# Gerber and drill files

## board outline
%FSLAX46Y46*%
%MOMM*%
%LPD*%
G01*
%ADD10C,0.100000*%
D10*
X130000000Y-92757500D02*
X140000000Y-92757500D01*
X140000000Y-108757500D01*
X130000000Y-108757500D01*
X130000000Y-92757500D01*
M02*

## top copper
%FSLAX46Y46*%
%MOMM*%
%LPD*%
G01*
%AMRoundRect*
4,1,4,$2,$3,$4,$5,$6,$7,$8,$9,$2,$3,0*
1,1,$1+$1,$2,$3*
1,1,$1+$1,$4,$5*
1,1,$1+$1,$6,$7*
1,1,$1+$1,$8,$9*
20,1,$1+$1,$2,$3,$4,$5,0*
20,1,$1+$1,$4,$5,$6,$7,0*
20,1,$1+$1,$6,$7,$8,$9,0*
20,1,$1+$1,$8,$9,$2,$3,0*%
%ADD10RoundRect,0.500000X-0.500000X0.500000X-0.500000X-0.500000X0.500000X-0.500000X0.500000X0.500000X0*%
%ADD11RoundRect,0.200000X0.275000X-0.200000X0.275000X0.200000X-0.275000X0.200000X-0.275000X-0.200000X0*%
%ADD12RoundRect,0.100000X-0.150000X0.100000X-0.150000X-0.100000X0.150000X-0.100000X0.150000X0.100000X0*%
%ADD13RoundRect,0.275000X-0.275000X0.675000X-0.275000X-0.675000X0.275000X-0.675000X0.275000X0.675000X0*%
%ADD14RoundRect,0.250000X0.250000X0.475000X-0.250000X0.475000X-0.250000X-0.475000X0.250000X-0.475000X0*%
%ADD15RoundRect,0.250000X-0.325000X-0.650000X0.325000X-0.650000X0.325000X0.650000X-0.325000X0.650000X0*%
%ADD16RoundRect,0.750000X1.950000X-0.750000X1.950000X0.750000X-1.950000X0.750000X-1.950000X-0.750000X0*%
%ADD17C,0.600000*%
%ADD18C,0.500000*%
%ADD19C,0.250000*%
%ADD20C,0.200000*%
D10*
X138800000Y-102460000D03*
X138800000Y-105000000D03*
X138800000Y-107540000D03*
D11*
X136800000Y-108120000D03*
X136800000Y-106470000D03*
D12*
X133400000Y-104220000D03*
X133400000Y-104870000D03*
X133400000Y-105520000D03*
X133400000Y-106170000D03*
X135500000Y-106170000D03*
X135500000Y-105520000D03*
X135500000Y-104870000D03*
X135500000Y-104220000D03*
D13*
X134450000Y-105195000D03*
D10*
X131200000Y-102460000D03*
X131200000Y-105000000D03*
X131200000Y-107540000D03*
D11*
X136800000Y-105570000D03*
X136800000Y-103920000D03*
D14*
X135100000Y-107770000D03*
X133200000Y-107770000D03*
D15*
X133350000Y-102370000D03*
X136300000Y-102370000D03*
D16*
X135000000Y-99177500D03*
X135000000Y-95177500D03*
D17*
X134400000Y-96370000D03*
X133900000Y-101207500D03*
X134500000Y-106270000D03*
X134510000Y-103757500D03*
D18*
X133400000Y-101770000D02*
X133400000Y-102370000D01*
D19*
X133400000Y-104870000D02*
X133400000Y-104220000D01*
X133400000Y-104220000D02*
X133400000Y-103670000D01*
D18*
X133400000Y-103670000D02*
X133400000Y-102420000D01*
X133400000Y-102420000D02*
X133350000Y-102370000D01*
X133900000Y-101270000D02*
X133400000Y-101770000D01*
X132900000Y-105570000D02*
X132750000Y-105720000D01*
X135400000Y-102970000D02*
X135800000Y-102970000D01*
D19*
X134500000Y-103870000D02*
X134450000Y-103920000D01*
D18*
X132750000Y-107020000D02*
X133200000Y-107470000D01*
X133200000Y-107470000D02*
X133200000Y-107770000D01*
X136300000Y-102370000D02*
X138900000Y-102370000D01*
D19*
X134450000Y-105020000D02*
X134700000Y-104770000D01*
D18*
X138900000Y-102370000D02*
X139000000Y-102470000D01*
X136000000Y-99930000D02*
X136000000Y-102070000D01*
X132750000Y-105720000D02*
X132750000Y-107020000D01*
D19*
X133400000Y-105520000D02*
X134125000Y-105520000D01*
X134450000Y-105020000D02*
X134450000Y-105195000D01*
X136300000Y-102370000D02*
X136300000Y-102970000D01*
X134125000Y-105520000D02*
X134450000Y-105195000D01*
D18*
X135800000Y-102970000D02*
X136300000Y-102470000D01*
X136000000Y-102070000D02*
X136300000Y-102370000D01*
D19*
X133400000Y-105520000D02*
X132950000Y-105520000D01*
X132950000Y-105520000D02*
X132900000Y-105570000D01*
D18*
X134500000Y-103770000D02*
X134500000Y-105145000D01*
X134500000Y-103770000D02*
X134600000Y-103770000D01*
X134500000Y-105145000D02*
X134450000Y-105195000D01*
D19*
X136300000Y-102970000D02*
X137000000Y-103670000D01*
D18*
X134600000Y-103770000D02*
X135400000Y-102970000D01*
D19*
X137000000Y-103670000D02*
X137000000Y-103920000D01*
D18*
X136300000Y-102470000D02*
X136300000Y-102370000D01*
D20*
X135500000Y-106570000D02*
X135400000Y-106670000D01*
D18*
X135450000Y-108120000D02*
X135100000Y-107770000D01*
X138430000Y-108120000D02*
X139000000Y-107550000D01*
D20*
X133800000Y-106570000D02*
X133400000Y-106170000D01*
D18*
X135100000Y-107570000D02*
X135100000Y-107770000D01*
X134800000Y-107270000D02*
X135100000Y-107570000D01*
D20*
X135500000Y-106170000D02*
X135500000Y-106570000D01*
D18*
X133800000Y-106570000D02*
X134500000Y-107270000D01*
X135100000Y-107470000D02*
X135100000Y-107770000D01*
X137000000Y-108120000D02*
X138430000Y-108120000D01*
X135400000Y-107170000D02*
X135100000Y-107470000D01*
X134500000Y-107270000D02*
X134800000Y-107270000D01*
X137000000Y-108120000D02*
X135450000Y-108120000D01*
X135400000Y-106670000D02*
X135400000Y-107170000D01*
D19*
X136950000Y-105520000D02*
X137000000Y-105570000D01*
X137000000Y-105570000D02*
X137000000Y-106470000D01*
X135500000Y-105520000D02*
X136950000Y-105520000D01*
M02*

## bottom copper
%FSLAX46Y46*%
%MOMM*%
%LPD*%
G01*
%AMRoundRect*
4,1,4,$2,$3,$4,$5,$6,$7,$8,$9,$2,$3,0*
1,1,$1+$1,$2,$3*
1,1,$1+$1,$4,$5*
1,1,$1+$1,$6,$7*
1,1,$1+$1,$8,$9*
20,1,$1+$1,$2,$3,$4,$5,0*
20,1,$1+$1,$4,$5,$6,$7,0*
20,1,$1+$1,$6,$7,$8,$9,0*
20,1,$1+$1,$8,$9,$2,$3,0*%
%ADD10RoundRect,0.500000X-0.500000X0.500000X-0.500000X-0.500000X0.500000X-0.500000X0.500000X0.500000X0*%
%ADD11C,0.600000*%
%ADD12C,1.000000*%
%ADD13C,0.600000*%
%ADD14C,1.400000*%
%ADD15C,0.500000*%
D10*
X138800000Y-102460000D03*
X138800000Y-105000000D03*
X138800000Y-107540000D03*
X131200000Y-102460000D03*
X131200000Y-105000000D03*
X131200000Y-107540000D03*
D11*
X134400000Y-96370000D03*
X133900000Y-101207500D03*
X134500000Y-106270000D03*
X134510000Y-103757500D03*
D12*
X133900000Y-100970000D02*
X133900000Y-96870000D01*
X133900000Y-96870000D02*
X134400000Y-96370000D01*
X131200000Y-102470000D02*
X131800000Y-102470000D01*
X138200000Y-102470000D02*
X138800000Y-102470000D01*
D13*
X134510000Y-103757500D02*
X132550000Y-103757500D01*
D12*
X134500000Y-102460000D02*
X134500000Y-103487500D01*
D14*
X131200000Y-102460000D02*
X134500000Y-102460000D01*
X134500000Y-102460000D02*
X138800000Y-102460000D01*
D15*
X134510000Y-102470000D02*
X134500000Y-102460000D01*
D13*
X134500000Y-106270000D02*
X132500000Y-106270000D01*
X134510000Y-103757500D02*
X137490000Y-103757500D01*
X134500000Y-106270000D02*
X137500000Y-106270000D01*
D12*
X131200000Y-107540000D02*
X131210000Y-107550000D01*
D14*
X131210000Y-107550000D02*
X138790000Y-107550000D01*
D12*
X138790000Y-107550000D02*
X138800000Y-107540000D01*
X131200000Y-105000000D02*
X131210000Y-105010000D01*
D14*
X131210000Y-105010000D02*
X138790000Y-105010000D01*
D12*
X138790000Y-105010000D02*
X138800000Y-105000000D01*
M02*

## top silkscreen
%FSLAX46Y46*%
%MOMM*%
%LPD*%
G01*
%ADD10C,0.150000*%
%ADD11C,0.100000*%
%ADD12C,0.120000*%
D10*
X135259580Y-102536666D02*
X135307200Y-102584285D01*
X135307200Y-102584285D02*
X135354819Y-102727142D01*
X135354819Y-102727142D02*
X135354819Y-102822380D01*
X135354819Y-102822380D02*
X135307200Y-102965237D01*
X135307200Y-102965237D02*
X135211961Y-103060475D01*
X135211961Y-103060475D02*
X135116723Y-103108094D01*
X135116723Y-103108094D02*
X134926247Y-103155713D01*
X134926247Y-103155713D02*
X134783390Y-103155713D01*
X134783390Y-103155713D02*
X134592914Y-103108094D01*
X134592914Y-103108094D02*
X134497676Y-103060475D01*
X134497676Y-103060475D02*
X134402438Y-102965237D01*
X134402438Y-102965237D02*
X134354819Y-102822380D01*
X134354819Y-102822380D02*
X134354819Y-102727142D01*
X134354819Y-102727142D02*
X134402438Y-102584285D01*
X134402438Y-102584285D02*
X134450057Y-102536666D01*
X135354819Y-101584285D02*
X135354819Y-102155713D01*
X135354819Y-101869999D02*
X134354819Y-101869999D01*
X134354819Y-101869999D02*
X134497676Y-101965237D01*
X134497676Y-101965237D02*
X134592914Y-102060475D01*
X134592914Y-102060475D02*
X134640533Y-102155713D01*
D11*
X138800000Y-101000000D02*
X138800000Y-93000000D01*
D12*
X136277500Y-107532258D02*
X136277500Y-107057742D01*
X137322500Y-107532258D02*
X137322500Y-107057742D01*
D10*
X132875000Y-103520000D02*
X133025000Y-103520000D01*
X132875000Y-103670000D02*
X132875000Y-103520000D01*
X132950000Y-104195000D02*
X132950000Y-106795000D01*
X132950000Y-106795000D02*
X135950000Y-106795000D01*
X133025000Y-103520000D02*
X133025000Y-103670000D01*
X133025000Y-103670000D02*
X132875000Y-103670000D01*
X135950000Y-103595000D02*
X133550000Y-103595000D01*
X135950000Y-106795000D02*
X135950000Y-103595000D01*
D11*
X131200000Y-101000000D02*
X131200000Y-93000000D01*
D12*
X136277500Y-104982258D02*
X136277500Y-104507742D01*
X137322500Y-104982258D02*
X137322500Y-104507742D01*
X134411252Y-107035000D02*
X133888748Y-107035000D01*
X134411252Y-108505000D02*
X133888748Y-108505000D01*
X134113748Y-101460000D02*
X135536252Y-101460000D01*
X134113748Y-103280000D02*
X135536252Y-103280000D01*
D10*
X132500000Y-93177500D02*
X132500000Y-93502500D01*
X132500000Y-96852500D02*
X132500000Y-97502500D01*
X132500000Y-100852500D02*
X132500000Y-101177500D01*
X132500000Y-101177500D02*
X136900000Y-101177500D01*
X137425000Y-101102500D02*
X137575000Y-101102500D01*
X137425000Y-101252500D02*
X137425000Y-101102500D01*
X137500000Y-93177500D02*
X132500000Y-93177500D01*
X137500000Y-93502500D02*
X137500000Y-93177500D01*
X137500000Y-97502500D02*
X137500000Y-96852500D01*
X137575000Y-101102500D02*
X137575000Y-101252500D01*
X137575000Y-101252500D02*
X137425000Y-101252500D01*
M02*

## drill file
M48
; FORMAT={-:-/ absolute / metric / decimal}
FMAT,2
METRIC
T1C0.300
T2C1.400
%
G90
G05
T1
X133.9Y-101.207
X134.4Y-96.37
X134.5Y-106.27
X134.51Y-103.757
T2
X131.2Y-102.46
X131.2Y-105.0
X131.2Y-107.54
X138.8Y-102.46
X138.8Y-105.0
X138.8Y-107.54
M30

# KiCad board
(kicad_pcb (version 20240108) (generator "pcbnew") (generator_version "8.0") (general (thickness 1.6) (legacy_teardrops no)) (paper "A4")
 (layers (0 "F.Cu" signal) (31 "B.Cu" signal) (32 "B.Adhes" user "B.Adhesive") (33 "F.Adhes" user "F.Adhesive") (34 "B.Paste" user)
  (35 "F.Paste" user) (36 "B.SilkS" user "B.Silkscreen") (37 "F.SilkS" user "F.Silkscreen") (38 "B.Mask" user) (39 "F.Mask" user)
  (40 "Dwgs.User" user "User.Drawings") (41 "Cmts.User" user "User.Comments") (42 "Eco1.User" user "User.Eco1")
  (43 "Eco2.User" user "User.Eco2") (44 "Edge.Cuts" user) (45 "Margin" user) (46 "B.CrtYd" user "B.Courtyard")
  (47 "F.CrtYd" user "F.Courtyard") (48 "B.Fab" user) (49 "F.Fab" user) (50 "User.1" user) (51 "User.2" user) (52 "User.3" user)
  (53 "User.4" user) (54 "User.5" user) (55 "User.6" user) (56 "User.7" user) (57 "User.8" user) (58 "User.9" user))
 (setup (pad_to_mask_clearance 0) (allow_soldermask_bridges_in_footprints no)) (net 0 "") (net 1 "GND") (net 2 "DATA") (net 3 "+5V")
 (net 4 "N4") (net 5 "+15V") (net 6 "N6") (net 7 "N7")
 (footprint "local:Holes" (layer "F.Cu") (at 138.8 105 -90)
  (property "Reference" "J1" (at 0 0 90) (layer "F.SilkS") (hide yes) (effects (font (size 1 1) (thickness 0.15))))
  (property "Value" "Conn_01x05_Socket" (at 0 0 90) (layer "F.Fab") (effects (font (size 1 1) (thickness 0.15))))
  (fp_line (start -4 0) (end -12 0) (stroke (width 0.1) (type solid)) (layer "F.SilkS"))
  (pad "1" thru_hole roundrect (at -2.54 0 270) (size 2 2) (drill 1.4) (layers "*.Cu" "*.Mask") (remove_unused_layers no)
   (roundrect_rratio 0.25) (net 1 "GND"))
  (pad "2" thru_hole roundrect (at 0 0 270) (size 2 2) (drill 1.4) (layers "*.Cu" "*.Mask") (remove_unused_layers no)
   (roundrect_rratio 0.25) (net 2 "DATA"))
  (pad "3" thru_hole roundrect (at 2.54 0 270) (size 2 2) (drill 1.4) (layers "*.Cu" "*.Mask") (remove_unused_layers no)
   (roundrect_rratio 0.25) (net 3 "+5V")))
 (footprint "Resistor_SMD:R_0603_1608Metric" (layer "F.Cu") (at 136.8 107.295 90)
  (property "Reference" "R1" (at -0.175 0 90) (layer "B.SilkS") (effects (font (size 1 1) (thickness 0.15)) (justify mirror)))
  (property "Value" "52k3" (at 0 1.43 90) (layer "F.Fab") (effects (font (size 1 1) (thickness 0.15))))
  (fp_line (start -0.237258 -0.5225) (end 0.237258 -0.5225) (stroke (width 0.12) (type solid)) (layer "F.SilkS"))
  (fp_line (start -0.237258 0.5225) (end 0.237258 0.5225) (stroke (width 0.12) (type solid)) (layer "F.SilkS"))
  (pad "1" smd roundrect (at -0.825 0 90) (size 0.8 0.95) (layers "F.Cu" "F.Paste" "F.Mask") (roundrect_rratio 0.25) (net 3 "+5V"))
  (pad "2" smd roundrect (at 0.825 0 90) (size 0.8 0.95) (layers "F.Cu" "F.Paste" "F.Mask") (roundrect_rratio 0.25) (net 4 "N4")))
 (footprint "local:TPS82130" (layer "F.Cu") (at 134.45 105.195 -90)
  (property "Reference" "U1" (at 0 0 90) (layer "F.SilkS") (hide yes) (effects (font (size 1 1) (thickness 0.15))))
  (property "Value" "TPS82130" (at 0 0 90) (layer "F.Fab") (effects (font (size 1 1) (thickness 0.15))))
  (fp_line (start -1.675 1.575) (end -1.675 1.425) (stroke (width 0.15) (type solid)) (layer "F.SilkS"))
  (fp_line (start -1.525 1.575) (end -1.675 1.575) (stroke (width 0.15) (type solid)) (layer "F.SilkS"))
  (fp_line (start -1 1.5) (end 1.6 1.5) (stroke (width 0.15) (type solid)) (layer "F.SilkS"))
  (fp_line (start 1.6 1.5) (end 1.6 -1.5) (stroke (width 0.15) (type solid)) (layer "F.SilkS"))
  (fp_line (start -1.675 1.425) (end -1.525 1.425) (stroke (width 0.15) (type solid)) (layer "F.SilkS"))
  (fp_line (start -1.525 1.425) (end -1.525 1.575) (stroke (width 0.15) (type solid)) (layer "F.SilkS"))
  (fp_line (start -1.6 -1.5) (end -1.6 0.9) (stroke (width 0.15) (type solid)) (layer "F.SilkS"))
  (fp_line (start 1.6 -1.5) (end -1.6 -1.5) (stroke (width 0.15) (type solid)) (layer "F.SilkS"))
  (pad "1" smd roundrect (at -0.975 1.05 270) (size 0.4 0.5) (layers "F.Cu" "F.Paste" "F.Mask") (roundrect_rratio 0.25) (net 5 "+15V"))
  (pad "2" smd roundrect (at -0.325 1.05 270) (size 0.4 0.5) (layers "F.Cu" "F.Paste" "F.Mask") (roundrect_rratio 0.25) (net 5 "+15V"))
  (pad "3" smd roundrect (at 0.325 1.05 270) (size 0.4 0.5) (layers "F.Cu" "F.Paste" "F.Mask") (roundrect_rratio 0.25) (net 1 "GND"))
  (pad "4" smd roundrect (at 0.975 1.05 270) (size 0.4 0.5) (layers "F.Cu" "F.Paste" "F.Mask") (roundrect_rratio 0.25) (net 3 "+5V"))
  (pad "5" smd roundrect (at 0.975 -1.05 270) (size 0.4 0.5) (layers "F.Cu" "F.Paste" "F.Mask") (roundrect_rratio 0.25) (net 3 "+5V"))
  (pad "6" smd roundrect (at 0.325 -1.05 270) (size 0.4 0.5) (layers "F.Cu" "F.Paste" "F.Mask") (roundrect_rratio 0.25) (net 4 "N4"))
  (pad "7" smd roundrect (at -0.325 -1.05 270) (size 0.4 0.5) (layers "F.Cu" "F.Paste" "F.Mask") (roundrect_rratio 0.25) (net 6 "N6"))
  (pad "8" smd roundrect (at -0.975 -1.05 270) (size 0.4 0.5) (layers "F.Cu" "F.Paste" "F.Mask") (roundrect_rratio 0.25) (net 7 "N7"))
  (pad "9" smd roundrect (at 0 0 270) (size 1.9 1.1) (layers "F.Cu" "F.Paste" "F.Mask") (roundrect_rratio 0.25) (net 1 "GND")))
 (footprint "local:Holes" (layer "F.Cu") (at 131.2 105 -90)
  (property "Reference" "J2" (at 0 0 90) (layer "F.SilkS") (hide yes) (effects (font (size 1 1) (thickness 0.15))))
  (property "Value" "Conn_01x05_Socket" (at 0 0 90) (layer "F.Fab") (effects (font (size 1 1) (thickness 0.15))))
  (fp_line (start -4 0) (end -12 0) (stroke (width 0.1) (type solid)) (layer "F.SilkS"))
  (pad "1" thru_hole roundrect (at -2.54 0 270) (size 2 2) (drill 1.4) (layers "*.Cu" "*.Mask") (remove_unused_layers no)
   (roundrect_rratio 0.25) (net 1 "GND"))
  (pad "2" thru_hole roundrect (at 0 0 270) (size 2 2) (drill 1.4) (layers "*.Cu" "*.Mask") (remove_unused_layers no)
   (roundrect_rratio 0.25) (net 2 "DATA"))
  (pad "3" thru_hole roundrect (at 2.54 0 270) (size 2 2) (drill 1.4) (layers "*.Cu" "*.Mask") (remove_unused_layers no)
   (roundrect_rratio 0.25) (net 3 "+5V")))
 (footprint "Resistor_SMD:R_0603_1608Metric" (layer "F.Cu") (at 136.8 104.745 90)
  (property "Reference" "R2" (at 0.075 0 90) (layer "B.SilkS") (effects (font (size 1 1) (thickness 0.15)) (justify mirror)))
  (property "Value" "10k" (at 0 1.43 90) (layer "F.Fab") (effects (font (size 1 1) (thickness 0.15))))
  (fp_line (start -0.237258 -0.5225) (end 0.237258 -0.5225) (stroke (width 0.12) (type solid)) (layer "F.SilkS"))
  (fp_line (start -0.237258 0.5225) (end 0.237258 0.5225) (stroke (width 0.12) (type solid)) (layer "F.SilkS"))
  (pad "1" smd roundrect (at -0.825 0 90) (size 0.8 0.95) (layers "F.Cu" "F.Paste" "F.Mask") (roundrect_rratio 0.25) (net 4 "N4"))
  (pad "2" smd roundrect (at 0.825 0 90) (size 0.8 0.95) (layers "F.Cu" "F.Paste" "F.Mask") (roundrect_rratio 0.25) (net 1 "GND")))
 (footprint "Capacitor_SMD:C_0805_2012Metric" (layer "F.Cu") (at 134.15 107.77 180)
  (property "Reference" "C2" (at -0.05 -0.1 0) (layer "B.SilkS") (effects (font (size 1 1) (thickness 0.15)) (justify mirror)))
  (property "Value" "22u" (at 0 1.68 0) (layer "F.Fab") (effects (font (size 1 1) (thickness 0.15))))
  (fp_line (start -0.261252 0.735) (end 0.261252 0.735) (stroke (width 0.12) (type solid)) (layer "F.SilkS"))
  (fp_line (start -0.261252 -0.735) (end 0.261252 -0.735) (stroke (width 0.12) (type solid)) (layer "F.SilkS"))
  (pad "1" smd roundrect (at -0.95 0 180) (size 1 1.45) (layers "F.Cu" "F.Paste" "F.Mask") (roundrect_rratio 0.25) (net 3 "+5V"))
  (pad "2" smd roundrect (at 0.95 0 180) (size 1 1.45) (layers "F.Cu" "F.Paste" "F.Mask") (roundrect_rratio 0.25) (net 1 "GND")))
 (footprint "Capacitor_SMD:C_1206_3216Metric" (layer "F.Cu") (at 134.825 102.37)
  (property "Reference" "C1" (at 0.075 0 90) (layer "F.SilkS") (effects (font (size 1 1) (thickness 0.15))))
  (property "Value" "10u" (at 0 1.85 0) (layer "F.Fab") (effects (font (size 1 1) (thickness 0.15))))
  (fp_line (start -0.711252 -0.91) (end 0.711252 -0.91) (stroke (width 0.12) (type solid)) (layer "F.SilkS"))
  (fp_line (start -0.711252 0.91) (end 0.711252 0.91) (stroke (width 0.12) (type solid)) (layer "F.SilkS"))
  (pad "1" smd roundrect (at -1.475 0) (size 1.15 1.8) (layers "F.Cu" "F.Paste" "F.Mask") (roundrect_rratio 0.217391) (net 5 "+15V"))
  (pad "2" smd roundrect (at 1.475 0) (size 1.15 1.8) (layers "F.Cu" "F.Paste" "F.Mask") (roundrect_rratio 0.217391) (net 1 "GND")))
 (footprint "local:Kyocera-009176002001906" (layer "F.Cu") (at 135 97.1775 90)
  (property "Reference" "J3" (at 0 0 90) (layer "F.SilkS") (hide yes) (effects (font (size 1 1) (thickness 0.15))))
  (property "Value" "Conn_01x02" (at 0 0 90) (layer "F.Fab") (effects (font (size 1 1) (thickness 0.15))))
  (fp_line (start 4 -2.5) (end 3.675 -2.5) (stroke (width 0.15) (type solid)) (layer "F.SilkS"))
  (fp_line (start 0.325 -2.5) (end -0.325 -2.5) (stroke (width 0.15) (type solid)) (layer "F.SilkS"))
  (fp_line (start -3.675 -2.5) (end -4 -2.5) (stroke (width 0.15) (type solid)) (layer "F.SilkS"))
  (fp_line (start -4 -2.5) (end -4 1.9) (stroke (width 0.15) (type solid)) (layer "F.SilkS"))
  (fp_line (start -3.925 2.425) (end -3.925 2.575) (stroke (width 0.15) (type solid)) (layer "F.SilkS"))
  (fp_line (start -4.075 2.425) (end -3.925 2.425) (stroke (width 0.15) (type solid)) (layer "F.SilkS"))
  (fp_line (start 4 2.5) (end 4 -2.5) (stroke (width 0.15) (type solid)) (layer "F.SilkS"))
  (fp_line (start 3.675 2.5) (end 4 2.5) (stroke (width 0.15) (type solid)) (layer "F.SilkS"))
  (fp_line (start -0.325 2.5) (end 0.325 2.5) (stroke (width 0.15) (type solid)) (layer "F.SilkS"))
  (fp_line (start -3.925 2.575) (end -4.075 2.575) (stroke (width 0.15) (type solid)) (layer "F.SilkS"))
  (fp_line (start -4.075 2.575) (end -4.075 2.425) (stroke (width 0.15) (type solid)) (layer "F.SilkS"))
  (pad "1" smd roundrect (at -2 0 90) (size 3 5.4) (layers "F.Cu" "F.Paste" "F.Mask") (roundrect_rratio 0.25) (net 1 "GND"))
  (pad "2" smd roundrect (at 2 0 90) (size 3 5.4) (layers "F.Cu" "F.Paste" "F.Mask") (roundrect_rratio 0.25) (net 5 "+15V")))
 (gr_rect (start 130 92.7575) (end 140 108.7575) (stroke (width 0.1) (type default)) (fill none) (layer "Edge.Cuts"))
 (segment (start 133.4 101.77) (end 133.4 102.37) (width 0.5) (layer "F.Cu") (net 5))
 (segment (start 133.4 104.87) (end 133.4 104.22) (width 0.25) (layer "F.Cu") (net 5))
 (segment (start 133.4 104.22) (end 133.4 103.67) (width 0.25) (layer "F.Cu") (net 5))
 (segment (start 133.4 103.67) (end 133.4 102.42) (width 0.5) (layer "F.Cu") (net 5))
 (segment (start 133.4 102.42) (end 133.35 102.37) (width 0.5) (layer "F.Cu") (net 5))
 (segment (start 133.9 101.27) (end 133.4 101.77) (width 0.5) (layer "F.Cu") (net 5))
 (via (at 134.4 96.37) (size 0.6) (drill 0.3) (layers "F.Cu" "B.Cu") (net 5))
 (via (at 133.9 101.2075) (size 0.6) (drill 0.3) (layers "F.Cu" "B.Cu") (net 5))
 (segment (start 133.9 100.97) (end 133.9 96.87) (width 1) (layer "B.Cu") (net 5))
 (segment (start 133.9 96.87) (end 134.4 96.37) (width 1) (layer "B.Cu") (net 5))
 (segment (start 132.9 105.57) (end 132.75 105.72) (width 0.5) (layer "F.Cu") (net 1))
 (segment (start 135.4 102.97) (end 135.8 102.97) (width 0.5) (layer "F.Cu") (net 1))
 (segment (start 134.5 103.87) (end 134.45 103.92) (width 0.25) (layer "F.Cu") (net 1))
 (segment (start 132.75 107.02) (end 133.2 107.47) (width 0.5) (layer "F.Cu") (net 1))
 (segment (start 133.2 107.47) (end 133.2 107.77) (width 0.5) (layer "F.Cu") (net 1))
 (segment (start 136.3 102.37) (end 138.9 102.37) (width 0.5) (layer "F.Cu") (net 1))
 (segment (start 134.45 105.02) (end 134.7 104.77) (width 0.25) (layer "F.Cu") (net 1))
 (segment (start 138.9 102.37) (end 139 102.47) (width 0.5) (layer "F.Cu") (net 1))
 (segment (start 136 99.93) (end 136 102.07) (width 0.5) (layer "F.Cu") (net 1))
 (segment (start 132.75 105.72) (end 132.75 107.02) (width 0.5) (layer "F.Cu") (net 1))
 (segment (start 133.4 105.52) (end 134.125 105.52) (width 0.25) (layer "F.Cu") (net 1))
 (segment (start 134.45 105.02) (end 134.45 105.195) (width 0.25) (layer "F.Cu") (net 1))
 (segment (start 136.3 102.37) (end 136.3 102.97) (width 0.25) (layer "F.Cu") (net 1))
 (segment (start 134.125 105.52) (end 134.45 105.195) (width 0.25) (layer "F.Cu") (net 1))
 (segment (start 135.8 102.97) (end 136.3 102.47) (width 0.5) (layer "F.Cu") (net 1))
 (segment (start 136 102.07) (end 136.3 102.37) (width 0.5) (layer "F.Cu") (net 1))
 (segment (start 133.4 105.52) (end 132.95 105.52) (width 0.25) (layer "F.Cu") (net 1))
 (segment (start 132.95 105.52) (end 132.9 105.57) (width 0.25) (layer "F.Cu") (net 1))
 (segment (start 134.5 103.77) (end 134.5 105.145) (width 0.5) (layer "F.Cu") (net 1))
 (segment (start 134.5 103.77) (end 134.6 103.77) (width 0.5) (layer "F.Cu") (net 1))
 (segment (start 134.5 105.145) (end 134.45 105.195) (width 0.5) (layer "F.Cu") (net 1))
 (segment (start 136.3 102.97) (end 137 103.67) (width 0.25) (layer "F.Cu") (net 1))
 (segment (start 134.6 103.77) (end 135.4 102.97) (width 0.5) (layer "F.Cu") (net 1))
 (segment (start 137 103.67) (end 137 103.92) (width 0.25) (layer "F.Cu") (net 1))
 (segment (start 136.3 102.47) (end 136.3 102.37) (width 0.5) (layer "F.Cu") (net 1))
 (via (at 134.5 106.27) (size 0.6) (drill 0.3) (layers "F.Cu" "B.Cu") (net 1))
 (via (at 134.51 103.7575) (size 0.6) (drill 0.3) (layers "F.Cu" "B.Cu") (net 1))
 (segment (start 131.2 102.47) (end 131.8 102.47) (width 1) (layer "B.Cu") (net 1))
 (segment (start 138.2 102.47) (end 138.8 102.47) (width 1) (layer "B.Cu") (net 1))
 (segment (start 134.51 103.7575) (end 132.55 103.7575) (width 0.6) (layer "B.Cu") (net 1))
 (segment (start 134.5 102.46) (end 134.5 103.4875) (width 1) (layer "B.Cu") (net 1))
 (segment (start 131.2 102.46) (end 134.5 102.46) (width 1.4) (layer "B.Cu") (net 1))
 (segment (start 134.5 102.46) (end 138.8 102.46) (width 1.4) (layer "B.Cu") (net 1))
 (segment (start 134.51 102.47) (end 134.5 102.46) (width 0.5) (layer "B.Cu") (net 1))
 (segment (start 134.5 106.27) (end 132.5 106.27) (width 0.6) (layer "B.Cu") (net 1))
 (segment (start 134.51 103.7575) (end 137.49 103.7575) (width 0.6) (layer "B.Cu") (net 1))
 (segment (start 134.5 106.27) (end 137.5 106.27) (width 0.6) (layer "B.Cu") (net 1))
 (segment (start 135.5 106.57) (end 135.4 106.67) (width 0.2) (layer "F.Cu") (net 3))
 (segment (start 135.45 108.12) (end 135.1 107.77) (width 0.5) (layer "F.Cu") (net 3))
 (segment (start 138.43 108.12) (end 139 107.55) (width 0.5) (layer "F.Cu") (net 3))
 (segment (start 133.8 106.57) (end 133.4 106.17) (width 0.2) (layer "F.Cu") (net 3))
 (segment (start 135.1 107.57) (end 135.1 107.77) (width 0.5) (layer "F.Cu") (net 3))
 (segment (start 134.8 107.27) (end 135.1 107.57) (width 0.5) (layer "F.Cu") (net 3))
 (segment (start 135.5 106.17) (end 135.5 106.57) (width 0.2) (layer "F.Cu") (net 3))
 (segment (start 133.8 106.57) (end 134.5 107.27) (width 0.5) (layer "F.Cu") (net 3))
 (segment (start 135.1 107.47) (end 135.1 107.77) (width 0.5) (layer "F.Cu") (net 3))
 (segment (start 137 108.12) (end 138.43 108.12) (width 0.5) (layer "F.Cu") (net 3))
 (segment (start 135.4 107.17) (end 135.1 107.47) (width 0.5) (layer "F.Cu") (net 3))
 (segment (start 134.5 107.27) (end 134.8 107.27) (width 0.5) (layer "F.Cu") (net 3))
 (segment (start 137 108.12) (end 135.45 108.12) (width 0.5) (layer "F.Cu") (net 3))
 (segment (start 135.4 106.67) (end 135.4 107.17) (width 0.5) (layer "F.Cu") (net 3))
 (segment (start 131.2 107.54) (end 131.21 107.55) (width 1) (layer "B.Cu") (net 3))
 (segment (start 131.21 107.55) (end 138.79 107.55) (width 1.4) (layer "B.Cu") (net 3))
 (segment (start 138.79 107.55) (end 138.8 107.54) (width 1) (layer "B.Cu") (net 3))
 (segment (start 136.95 105.52) (end 137 105.57) (width 0.25) (layer "F.Cu") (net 4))
 (segment (start 137 105.57) (end 137 106.47) (width 0.25) (layer "F.Cu") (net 4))
 (segment (start 135.5 105.52) (end 136.95 105.52) (width 0.25) (layer "F.Cu") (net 4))
 (segment (start 131.2 105) (end 131.21 105.01) (width 1) (layer "B.Cu") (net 2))
 (segment (start 131.21 105.01) (end 138.79 105.01) (width 1.4) (layer "B.Cu") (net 2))
 (segment (start 138.79 105.01) (end 138.8 105) (width 1) (layer "B.Cu") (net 2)))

